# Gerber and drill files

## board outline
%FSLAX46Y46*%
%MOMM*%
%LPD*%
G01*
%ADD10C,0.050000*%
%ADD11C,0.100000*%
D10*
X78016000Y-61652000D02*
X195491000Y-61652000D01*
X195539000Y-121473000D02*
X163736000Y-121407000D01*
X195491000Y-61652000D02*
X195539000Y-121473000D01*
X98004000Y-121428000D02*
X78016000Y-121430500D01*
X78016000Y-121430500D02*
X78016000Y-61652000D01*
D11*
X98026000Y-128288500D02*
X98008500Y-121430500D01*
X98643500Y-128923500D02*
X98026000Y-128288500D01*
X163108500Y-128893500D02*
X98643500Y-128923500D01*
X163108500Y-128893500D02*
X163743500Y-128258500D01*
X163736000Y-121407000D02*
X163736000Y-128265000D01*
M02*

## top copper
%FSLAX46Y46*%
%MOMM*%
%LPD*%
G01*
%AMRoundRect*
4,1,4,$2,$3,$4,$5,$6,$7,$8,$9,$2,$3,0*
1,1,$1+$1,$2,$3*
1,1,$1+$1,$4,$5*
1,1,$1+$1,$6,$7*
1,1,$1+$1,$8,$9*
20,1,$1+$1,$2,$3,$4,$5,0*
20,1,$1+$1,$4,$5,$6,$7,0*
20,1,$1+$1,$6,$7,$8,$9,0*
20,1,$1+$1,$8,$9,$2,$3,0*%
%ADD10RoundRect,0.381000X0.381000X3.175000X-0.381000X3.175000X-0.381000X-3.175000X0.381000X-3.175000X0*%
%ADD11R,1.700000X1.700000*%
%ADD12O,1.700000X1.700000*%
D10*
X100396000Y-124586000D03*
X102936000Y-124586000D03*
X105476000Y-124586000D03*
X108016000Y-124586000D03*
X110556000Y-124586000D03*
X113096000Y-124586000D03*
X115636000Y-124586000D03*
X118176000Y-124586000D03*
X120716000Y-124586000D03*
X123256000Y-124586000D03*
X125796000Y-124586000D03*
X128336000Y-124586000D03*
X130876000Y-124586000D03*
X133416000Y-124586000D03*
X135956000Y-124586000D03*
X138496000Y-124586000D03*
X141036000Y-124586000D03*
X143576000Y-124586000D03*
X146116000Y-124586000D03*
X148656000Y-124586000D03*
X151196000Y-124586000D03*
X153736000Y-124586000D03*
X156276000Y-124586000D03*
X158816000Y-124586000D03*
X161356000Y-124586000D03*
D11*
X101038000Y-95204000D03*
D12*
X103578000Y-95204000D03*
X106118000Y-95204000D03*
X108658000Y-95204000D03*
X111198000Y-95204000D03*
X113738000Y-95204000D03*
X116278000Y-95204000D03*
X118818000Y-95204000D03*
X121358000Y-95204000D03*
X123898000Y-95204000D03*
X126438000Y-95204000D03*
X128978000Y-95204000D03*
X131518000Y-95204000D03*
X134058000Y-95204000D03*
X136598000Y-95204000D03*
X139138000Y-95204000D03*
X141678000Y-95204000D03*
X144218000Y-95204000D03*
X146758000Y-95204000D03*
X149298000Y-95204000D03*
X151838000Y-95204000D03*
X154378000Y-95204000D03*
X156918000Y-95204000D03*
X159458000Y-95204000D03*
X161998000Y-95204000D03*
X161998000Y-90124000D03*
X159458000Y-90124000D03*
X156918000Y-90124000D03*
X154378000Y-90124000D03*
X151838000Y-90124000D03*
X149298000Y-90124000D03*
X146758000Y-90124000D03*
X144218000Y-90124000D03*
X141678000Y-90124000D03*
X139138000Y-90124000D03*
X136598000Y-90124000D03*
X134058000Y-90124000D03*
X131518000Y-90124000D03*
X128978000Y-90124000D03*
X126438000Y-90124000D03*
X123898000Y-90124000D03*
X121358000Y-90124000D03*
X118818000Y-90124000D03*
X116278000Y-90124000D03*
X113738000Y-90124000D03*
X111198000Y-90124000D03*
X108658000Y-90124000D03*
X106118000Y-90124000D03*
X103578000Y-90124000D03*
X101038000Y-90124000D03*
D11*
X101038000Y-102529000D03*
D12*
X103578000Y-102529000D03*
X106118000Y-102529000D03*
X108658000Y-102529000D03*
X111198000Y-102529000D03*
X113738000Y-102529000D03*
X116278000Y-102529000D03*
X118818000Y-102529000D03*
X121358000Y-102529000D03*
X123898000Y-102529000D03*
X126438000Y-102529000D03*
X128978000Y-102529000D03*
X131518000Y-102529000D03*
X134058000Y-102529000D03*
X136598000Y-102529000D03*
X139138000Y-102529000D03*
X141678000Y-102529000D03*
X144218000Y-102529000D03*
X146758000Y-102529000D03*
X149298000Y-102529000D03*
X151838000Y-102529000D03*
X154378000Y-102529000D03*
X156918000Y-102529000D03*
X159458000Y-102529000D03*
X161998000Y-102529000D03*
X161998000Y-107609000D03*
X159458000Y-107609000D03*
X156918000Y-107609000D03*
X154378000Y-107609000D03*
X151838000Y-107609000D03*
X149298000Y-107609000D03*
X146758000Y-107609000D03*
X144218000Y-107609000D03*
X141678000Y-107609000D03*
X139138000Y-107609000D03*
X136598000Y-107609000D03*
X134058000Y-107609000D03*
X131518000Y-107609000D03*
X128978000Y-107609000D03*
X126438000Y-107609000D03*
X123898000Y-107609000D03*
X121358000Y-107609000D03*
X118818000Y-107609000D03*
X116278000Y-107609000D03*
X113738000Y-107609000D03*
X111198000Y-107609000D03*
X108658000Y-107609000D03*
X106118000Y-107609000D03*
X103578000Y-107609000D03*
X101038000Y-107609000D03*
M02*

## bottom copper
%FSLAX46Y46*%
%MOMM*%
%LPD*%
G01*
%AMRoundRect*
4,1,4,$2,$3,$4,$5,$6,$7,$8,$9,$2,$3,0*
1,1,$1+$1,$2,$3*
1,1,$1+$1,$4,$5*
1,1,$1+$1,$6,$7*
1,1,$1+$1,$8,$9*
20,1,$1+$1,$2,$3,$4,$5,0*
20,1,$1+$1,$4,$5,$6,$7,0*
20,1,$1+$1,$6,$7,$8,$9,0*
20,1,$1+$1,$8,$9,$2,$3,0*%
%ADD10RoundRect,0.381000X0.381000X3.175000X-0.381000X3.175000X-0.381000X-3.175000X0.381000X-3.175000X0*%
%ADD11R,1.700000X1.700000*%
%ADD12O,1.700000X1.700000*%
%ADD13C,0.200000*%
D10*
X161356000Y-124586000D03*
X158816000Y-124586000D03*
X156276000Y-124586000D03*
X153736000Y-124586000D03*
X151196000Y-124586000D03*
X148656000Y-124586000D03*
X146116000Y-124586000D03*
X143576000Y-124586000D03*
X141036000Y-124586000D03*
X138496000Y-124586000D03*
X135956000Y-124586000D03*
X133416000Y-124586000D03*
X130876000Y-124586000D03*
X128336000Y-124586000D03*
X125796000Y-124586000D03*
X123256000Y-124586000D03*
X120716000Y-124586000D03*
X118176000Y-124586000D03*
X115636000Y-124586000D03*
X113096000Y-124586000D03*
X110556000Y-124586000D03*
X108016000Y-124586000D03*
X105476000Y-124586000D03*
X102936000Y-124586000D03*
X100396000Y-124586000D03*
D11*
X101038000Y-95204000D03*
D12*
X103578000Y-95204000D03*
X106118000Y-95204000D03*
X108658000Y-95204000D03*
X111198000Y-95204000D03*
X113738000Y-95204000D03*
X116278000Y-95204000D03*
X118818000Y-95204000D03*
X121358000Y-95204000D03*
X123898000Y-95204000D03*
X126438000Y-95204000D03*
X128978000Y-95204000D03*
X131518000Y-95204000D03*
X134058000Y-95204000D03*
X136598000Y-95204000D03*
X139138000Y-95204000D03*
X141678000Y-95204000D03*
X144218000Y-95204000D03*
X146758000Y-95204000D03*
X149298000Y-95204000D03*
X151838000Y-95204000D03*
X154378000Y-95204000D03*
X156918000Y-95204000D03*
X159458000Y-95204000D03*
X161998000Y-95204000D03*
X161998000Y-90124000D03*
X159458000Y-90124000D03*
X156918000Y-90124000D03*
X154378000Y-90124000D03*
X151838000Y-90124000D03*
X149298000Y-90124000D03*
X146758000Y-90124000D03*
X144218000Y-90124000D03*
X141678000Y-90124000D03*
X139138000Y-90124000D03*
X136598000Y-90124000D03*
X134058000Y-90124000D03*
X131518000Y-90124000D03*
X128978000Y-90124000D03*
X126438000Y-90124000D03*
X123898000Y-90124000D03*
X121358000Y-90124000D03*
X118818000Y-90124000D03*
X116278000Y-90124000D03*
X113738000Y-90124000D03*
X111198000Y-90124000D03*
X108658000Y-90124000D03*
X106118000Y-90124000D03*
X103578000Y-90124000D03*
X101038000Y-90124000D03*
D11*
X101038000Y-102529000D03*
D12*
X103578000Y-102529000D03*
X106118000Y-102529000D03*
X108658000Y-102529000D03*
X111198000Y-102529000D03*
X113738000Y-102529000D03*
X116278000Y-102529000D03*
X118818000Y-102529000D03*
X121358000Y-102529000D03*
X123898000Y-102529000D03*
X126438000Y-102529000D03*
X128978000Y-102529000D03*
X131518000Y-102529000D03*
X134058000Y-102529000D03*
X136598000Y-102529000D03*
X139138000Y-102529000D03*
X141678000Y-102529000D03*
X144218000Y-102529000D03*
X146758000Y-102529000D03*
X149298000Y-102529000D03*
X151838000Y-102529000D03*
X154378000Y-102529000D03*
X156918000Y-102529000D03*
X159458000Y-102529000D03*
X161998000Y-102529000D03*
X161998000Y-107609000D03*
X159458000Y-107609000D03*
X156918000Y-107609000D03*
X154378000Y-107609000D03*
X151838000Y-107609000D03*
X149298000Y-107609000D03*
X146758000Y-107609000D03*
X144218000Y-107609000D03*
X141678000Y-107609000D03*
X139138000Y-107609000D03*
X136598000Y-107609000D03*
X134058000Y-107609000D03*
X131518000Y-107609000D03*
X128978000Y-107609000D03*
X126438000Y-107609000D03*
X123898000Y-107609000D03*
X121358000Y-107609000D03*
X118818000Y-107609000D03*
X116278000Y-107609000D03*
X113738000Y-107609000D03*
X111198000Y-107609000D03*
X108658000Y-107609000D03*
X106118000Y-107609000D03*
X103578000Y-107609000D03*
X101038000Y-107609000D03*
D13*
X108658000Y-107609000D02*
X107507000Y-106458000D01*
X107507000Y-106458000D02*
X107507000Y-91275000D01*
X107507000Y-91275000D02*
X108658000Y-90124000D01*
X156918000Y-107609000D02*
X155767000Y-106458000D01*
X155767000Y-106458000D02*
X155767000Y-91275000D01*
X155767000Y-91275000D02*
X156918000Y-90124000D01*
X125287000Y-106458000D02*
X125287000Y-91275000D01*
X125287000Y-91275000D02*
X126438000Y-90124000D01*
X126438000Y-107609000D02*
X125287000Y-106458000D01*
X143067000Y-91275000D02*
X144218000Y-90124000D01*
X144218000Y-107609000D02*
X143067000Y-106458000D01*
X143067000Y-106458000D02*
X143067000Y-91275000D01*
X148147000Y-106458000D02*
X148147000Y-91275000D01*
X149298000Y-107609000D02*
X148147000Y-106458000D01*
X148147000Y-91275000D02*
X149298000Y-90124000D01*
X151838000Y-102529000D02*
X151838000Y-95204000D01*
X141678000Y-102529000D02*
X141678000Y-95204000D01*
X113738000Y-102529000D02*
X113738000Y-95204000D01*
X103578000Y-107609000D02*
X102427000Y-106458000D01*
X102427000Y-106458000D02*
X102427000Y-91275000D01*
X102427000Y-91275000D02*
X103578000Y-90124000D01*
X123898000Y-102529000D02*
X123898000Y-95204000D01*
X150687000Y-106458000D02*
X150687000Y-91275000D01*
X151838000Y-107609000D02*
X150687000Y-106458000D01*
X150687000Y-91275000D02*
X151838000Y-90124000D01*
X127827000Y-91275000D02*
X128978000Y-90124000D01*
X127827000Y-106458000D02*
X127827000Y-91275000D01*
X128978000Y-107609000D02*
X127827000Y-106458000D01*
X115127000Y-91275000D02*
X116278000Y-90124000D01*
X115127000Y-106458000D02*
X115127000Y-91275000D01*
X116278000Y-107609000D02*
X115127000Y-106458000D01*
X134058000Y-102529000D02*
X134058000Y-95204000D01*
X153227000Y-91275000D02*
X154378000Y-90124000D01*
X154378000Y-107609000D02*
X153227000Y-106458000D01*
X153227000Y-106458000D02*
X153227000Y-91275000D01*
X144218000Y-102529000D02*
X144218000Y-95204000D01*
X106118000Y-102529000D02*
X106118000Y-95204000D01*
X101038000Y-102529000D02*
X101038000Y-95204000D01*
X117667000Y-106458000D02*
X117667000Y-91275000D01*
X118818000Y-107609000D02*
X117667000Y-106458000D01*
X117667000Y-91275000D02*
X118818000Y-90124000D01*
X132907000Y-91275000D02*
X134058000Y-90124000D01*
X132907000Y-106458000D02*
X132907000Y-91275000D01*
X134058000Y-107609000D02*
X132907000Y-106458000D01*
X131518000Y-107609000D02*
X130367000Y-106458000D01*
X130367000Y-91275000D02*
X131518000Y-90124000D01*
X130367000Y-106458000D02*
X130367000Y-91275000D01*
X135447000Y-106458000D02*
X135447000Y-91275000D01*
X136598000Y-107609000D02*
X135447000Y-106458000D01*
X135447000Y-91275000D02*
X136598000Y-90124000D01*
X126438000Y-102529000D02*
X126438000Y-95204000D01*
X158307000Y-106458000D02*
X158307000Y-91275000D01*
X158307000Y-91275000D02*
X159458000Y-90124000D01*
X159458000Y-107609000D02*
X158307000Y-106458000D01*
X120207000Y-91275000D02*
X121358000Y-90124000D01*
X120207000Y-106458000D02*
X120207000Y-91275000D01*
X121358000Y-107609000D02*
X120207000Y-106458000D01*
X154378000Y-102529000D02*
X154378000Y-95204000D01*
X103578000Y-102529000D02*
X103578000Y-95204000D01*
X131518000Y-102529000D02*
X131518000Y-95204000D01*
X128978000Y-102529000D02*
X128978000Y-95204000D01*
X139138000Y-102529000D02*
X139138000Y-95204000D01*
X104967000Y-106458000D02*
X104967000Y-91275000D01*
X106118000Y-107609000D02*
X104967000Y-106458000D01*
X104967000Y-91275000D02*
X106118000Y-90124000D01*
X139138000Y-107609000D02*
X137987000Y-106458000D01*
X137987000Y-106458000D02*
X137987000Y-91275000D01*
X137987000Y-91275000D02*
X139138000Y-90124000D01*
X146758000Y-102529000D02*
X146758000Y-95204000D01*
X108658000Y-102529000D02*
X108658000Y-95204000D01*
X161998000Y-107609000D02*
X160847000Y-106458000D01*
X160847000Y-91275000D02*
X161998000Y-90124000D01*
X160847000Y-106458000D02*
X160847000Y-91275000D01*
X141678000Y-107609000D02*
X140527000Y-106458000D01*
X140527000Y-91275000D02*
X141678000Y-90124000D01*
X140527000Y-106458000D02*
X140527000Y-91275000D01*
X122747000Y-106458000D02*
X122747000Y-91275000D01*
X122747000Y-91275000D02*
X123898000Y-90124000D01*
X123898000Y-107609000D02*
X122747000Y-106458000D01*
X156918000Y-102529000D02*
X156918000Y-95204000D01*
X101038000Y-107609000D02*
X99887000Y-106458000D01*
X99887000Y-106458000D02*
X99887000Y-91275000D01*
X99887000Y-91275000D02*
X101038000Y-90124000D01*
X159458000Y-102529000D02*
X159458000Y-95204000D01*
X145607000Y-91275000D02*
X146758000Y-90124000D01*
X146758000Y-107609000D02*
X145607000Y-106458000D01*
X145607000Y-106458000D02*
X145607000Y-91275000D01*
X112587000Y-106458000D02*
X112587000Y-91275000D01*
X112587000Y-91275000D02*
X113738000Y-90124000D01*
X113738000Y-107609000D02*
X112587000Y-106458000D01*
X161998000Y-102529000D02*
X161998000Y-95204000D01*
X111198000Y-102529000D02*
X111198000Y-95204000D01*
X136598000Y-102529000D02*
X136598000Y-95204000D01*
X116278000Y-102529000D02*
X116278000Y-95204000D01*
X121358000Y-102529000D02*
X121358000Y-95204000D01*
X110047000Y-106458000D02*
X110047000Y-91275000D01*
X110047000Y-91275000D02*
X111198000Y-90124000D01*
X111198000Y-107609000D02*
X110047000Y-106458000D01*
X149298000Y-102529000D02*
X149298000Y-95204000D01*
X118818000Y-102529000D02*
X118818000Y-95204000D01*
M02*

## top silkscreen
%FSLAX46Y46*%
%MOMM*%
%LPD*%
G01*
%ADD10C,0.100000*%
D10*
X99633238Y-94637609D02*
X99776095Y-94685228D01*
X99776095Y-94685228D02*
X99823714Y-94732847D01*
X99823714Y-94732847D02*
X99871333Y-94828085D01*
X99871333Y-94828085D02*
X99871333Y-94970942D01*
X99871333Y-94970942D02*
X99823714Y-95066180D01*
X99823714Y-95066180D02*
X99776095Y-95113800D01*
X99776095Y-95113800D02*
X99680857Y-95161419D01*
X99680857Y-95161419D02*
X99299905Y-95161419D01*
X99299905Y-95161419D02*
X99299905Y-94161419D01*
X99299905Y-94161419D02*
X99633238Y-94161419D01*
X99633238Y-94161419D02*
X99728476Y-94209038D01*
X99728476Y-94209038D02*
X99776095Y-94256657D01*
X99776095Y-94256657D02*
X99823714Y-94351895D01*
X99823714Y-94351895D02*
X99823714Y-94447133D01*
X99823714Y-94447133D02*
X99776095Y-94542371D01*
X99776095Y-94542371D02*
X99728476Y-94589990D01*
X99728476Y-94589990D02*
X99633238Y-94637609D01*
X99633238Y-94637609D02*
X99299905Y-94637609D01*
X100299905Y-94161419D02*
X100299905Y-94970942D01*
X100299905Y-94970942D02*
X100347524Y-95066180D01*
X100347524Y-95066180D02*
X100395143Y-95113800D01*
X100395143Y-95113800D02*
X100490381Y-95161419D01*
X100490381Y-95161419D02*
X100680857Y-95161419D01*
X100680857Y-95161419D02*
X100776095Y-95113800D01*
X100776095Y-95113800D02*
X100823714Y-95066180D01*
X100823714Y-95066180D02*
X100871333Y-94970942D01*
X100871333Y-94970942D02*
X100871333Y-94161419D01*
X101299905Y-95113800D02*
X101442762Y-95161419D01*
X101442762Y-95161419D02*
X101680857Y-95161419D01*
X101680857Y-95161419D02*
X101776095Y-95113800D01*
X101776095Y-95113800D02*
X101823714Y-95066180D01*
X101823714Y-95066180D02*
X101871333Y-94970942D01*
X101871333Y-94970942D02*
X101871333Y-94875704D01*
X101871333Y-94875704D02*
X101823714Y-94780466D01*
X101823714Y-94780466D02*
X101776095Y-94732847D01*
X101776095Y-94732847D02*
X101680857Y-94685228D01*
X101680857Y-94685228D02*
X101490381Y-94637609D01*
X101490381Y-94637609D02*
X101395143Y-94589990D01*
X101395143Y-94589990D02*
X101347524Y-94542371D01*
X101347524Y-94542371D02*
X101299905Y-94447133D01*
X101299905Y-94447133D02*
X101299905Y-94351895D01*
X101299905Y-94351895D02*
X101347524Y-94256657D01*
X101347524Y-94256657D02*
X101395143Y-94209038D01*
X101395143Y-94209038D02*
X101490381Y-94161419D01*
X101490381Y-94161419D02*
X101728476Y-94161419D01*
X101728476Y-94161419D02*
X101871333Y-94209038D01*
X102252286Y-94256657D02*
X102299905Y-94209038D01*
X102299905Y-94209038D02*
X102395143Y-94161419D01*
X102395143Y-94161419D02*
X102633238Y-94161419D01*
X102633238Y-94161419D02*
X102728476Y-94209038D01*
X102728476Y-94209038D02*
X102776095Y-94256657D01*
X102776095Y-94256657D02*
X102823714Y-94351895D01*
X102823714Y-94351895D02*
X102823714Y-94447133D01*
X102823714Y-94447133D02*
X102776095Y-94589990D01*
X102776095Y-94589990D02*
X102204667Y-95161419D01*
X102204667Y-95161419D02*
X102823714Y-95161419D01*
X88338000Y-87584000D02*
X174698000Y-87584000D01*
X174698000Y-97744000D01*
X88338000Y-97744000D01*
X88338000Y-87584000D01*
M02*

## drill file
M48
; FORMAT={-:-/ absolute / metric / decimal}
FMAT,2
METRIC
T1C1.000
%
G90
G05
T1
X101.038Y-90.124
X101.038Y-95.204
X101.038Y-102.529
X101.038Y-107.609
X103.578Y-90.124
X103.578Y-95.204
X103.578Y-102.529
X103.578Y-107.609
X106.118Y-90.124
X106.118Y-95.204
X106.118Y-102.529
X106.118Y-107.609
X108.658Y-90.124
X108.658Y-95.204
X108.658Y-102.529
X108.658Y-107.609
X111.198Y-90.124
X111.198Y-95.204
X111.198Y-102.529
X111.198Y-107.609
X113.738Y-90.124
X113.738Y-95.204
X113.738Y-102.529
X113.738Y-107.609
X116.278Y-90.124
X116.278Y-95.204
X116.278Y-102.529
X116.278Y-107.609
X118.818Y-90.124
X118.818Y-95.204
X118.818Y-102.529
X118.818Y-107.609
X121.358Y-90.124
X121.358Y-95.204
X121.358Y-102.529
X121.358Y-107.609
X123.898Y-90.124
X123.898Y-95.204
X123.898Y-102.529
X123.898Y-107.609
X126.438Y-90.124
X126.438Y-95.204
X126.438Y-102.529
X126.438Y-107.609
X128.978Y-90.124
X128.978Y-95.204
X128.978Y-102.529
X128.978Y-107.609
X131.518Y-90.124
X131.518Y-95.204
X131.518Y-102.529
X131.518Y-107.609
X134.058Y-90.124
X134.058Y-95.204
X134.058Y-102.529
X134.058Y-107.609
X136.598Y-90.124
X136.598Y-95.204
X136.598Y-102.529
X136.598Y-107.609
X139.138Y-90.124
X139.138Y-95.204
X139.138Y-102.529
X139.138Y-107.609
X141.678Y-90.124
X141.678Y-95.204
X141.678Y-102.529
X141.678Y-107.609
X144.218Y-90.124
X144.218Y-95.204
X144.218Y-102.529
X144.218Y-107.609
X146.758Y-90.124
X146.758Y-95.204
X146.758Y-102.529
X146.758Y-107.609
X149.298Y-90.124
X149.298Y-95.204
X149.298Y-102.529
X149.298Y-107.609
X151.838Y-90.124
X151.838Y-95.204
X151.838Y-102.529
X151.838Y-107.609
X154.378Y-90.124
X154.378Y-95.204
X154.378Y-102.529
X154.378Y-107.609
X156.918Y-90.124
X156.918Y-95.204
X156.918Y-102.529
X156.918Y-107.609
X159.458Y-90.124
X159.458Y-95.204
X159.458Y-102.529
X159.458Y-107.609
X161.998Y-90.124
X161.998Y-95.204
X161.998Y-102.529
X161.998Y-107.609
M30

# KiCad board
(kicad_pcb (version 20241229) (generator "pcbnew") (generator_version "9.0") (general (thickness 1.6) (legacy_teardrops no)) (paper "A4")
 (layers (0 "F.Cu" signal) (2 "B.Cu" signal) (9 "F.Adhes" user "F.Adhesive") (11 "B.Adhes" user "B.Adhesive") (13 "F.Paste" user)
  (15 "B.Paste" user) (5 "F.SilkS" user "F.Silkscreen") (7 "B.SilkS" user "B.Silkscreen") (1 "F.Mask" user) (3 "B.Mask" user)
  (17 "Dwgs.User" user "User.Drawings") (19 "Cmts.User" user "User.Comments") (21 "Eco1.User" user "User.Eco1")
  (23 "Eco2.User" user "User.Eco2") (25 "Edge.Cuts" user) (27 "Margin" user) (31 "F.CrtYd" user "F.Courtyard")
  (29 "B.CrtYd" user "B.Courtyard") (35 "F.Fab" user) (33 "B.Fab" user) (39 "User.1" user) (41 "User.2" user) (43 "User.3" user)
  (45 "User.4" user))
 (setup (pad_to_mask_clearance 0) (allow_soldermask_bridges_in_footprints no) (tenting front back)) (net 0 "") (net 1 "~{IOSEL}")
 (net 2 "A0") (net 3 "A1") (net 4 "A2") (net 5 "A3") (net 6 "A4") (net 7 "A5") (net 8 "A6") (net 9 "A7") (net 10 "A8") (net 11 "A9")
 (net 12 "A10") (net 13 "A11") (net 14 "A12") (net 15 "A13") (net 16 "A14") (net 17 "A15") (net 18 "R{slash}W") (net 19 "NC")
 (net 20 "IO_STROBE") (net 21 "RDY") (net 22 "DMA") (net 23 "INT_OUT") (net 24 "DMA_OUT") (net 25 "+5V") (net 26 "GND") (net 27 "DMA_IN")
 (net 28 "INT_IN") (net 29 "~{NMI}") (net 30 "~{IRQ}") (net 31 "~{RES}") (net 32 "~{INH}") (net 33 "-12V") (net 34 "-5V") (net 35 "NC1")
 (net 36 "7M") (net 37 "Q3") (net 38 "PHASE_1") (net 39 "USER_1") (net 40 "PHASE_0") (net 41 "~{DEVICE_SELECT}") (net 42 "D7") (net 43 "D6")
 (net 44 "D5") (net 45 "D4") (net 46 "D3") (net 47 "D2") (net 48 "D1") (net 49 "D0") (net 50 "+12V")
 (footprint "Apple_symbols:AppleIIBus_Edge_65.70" (layer "F.Cu") (at 130.876 124.586)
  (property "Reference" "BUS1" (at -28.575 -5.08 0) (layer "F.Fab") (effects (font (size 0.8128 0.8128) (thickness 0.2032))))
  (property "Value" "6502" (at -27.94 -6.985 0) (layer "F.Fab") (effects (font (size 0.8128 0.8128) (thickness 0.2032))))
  (fp_line (start -32.85 3.7025) (end -32.8675 -3.1555) (stroke (width 0.1) (type solid)) (layer "Edge.Cuts"))
  (fp_line (start -32.2325 4.3375) (end -32.85 3.7025) (stroke (width 0.1) (type default)) (layer "Edge.Cuts"))
  (fp_line (start 32.2325 4.3075) (end -32.2325 4.3375) (stroke (width 0.1) (type solid)) (layer "Edge.Cuts"))
  (fp_line (start 32.2325 4.3075) (end 32.8675 3.6725) (stroke (width 0.1) (type default)) (layer "Edge.Cuts"))
  (fp_line (start 32.86 -3.179) (end 32.86 3.679) (stroke (width 0.1) (type solid)) (layer "Edge.Cuts"))
  (pad "1" connect roundrect (at -30.48 0 180) (size 1.524 7.112) (layers "F.Cu" "F.Mask") (roundrect_rratio 0.25) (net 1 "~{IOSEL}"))
  (pad "2" connect roundrect (at -27.94 0 180) (size 1.524 7.112) (layers "F.Cu" "F.Mask") (roundrect_rratio 0.25) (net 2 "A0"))
  (pad "3" connect roundrect (at -25.4 0 180) (size 1.524 7.112) (layers "F.Cu" "F.Mask") (roundrect_rratio 0.25) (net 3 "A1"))
  (pad "4" connect roundrect (at -22.86 0 180) (size 1.524 7.112) (layers "F.Cu" "F.Mask") (roundrect_rratio 0.25) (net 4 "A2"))
  (pad "5" connect roundrect (at -20.32 0 180) (size 1.524 7.112) (layers "F.Cu" "F.Mask") (roundrect_rratio 0.25) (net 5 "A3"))
  (pad "6" connect roundrect (at -17.78 0 180) (size 1.524 7.112) (layers "F.Cu" "F.Mask") (roundrect_rratio 0.25) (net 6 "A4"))
  (pad "7" connect roundrect (at -15.24 0 180) (size 1.524 7.112) (layers "F.Cu" "F.Mask") (roundrect_rratio 0.25) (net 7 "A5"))
  (pad "8" connect roundrect (at -12.7 0 180) (size 1.524 7.112) (layers "F.Cu" "F.Mask") (roundrect_rratio 0.25) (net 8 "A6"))
  (pad "9" connect roundrect (at -10.16 0 180) (size 1.524 7.112) (layers "F.Cu" "F.Mask") (roundrect_rratio 0.25) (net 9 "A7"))
  (pad "10" connect roundrect (at -7.62 0 180) (size 1.524 7.112) (layers "F.Cu" "F.Mask") (roundrect_rratio 0.25) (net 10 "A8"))
  (pad "11" connect roundrect (at -5.08 0 180) (size 1.524 7.112) (layers "F.Cu" "F.Mask") (roundrect_rratio 0.25) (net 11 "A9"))
  (pad "12" connect roundrect (at -2.54 0 180) (size 1.524 7.112) (layers "F.Cu" "F.Mask") (roundrect_rratio 0.25) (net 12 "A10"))
  (pad "13" connect roundrect (at 0 0 180) (size 1.524 7.112) (layers "F.Cu" "F.Mask") (roundrect_rratio 0.25) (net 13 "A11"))
  (pad "14" connect roundrect (at 2.54 0 180) (size 1.524 7.112) (layers "F.Cu" "F.Mask") (roundrect_rratio 0.25) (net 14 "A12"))
  (pad "15" connect roundrect (at 5.08 0 180) (size 1.524 7.112) (layers "F.Cu" "F.Mask") (roundrect_rratio 0.25) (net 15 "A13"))
  (pad "16" connect roundrect (at 7.62 0 180) (size 1.524 7.112) (layers "F.Cu" "F.Mask") (roundrect_rratio 0.25) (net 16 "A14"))
  (pad "17" connect roundrect (at 10.16 0 180) (size 1.524 7.112) (layers "F.Cu" "F.Mask") (roundrect_rratio 0.25) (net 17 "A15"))
  (pad "18" connect roundrect (at 12.7 0 180) (size 1.524 7.112) (layers "F.Cu" "F.Mask") (roundrect_rratio 0.25) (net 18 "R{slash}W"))
  (pad "19" connect roundrect (at 15.24 0 180) (size 1.524 7.112) (layers "F.Cu" "F.Mask") (roundrect_rratio 0.25) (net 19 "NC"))
  (pad "20" connect roundrect (at 17.78 0 180) (size 1.524 7.112) (layers "F.Cu" "F.Mask") (roundrect_rratio 0.25) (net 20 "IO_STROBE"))
  (pad "21" connect roundrect (at 20.32 0 180) (size 1.524 7.112) (layers "F.Cu" "F.Mask") (roundrect_rratio 0.25) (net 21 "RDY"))
  (pad "22" connect roundrect (at 22.86 0 180) (size 1.524 7.112) (layers "F.Cu" "F.Mask") (roundrect_rratio 0.25) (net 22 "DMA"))
  (pad "23" connect roundrect (at 25.4 0 180) (size 1.524 7.112) (layers "F.Cu" "F.Mask") (roundrect_rratio 0.25) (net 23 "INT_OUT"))
  (pad "24" connect roundrect (at 27.94 0 180) (size 1.524 7.112) (layers "F.Cu" "F.Mask") (roundrect_rratio 0.25) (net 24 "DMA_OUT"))
  (pad "25" connect roundrect (at 30.48 0 180) (size 1.524 7.112) (layers "F.Cu" "F.Mask") (roundrect_rratio 0.25) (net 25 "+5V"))
  (pad "26" connect roundrect (at 30.48 0 180) (size 1.524 7.112) (layers "B.Cu" "B.Mask") (roundrect_rratio 0.25) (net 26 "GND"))
  (pad "27" connect roundrect (at 27.94 0 180) (size 1.524 7.112) (layers "B.Cu" "B.Mask") (roundrect_rratio 0.25) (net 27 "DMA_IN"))
  (pad "28" connect roundrect (at 25.4 0 180) (size 1.524 7.112) (layers "B.Cu" "B.Mask") (roundrect_rratio 0.25) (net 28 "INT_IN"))
  (pad "29" connect roundrect (at 22.86 0 180) (size 1.524 7.112) (layers "B.Cu" "B.Mask") (roundrect_rratio 0.25) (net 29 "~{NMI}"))
  (pad "30" connect roundrect (at 20.32 0 180) (size 1.524 7.112) (layers "B.Cu" "B.Mask") (roundrect_rratio 0.25) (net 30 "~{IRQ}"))
  (pad "31" connect roundrect (at 17.78 0 180) (size 1.524 7.112) (layers "B.Cu" "B.Mask") (roundrect_rratio 0.25) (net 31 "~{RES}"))
  (pad "32" connect roundrect (at 15.24 0 180) (size 1.524 7.112) (layers "B.Cu" "B.Mask") (roundrect_rratio 0.25) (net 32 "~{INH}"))
  (pad "33" connect roundrect (at 12.7 0 180) (size 1.524 7.112) (layers "B.Cu" "B.Mask") (roundrect_rratio 0.25) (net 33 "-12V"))
  (pad "34" connect roundrect (at 10.16 0 180) (size 1.524 7.112) (layers "B.Cu" "B.Mask") (roundrect_rratio 0.25) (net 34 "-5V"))
  (pad "35" connect roundrect (at 7.62 0 180) (size 1.524 7.112) (layers "B.Cu" "B.Mask") (roundrect_rratio 0.25) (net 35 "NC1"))
  (pad "36" connect roundrect (at 5.08 0 180) (size 1.524 7.112) (layers "B.Cu" "B.Mask") (roundrect_rratio 0.25) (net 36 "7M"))
  (pad "37" connect roundrect (at 2.54 0 180) (size 1.524 7.112) (layers "B.Cu" "B.Mask") (roundrect_rratio 0.25) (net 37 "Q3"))
  (pad "38" connect roundrect (at 0 0 180) (size 1.524 7.112) (layers "B.Cu" "B.Mask") (roundrect_rratio 0.25) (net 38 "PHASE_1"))
  (pad "39" connect roundrect (at -2.54 0 180) (size 1.524 7.112) (layers "B.Cu" "B.Mask") (roundrect_rratio 0.25) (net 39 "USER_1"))
  (pad "40" connect roundrect (at -5.08 0 180) (size 1.524 7.112) (layers "B.Cu" "B.Mask") (roundrect_rratio 0.25) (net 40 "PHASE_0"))
  (pad "41" connect roundrect (at -7.62 0 180) (size 1.524 7.112) (layers "B.Cu" "B.Mask") (roundrect_rratio 0.25)
   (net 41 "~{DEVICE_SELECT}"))
  (pad "42" connect roundrect (at -10.16 0 180) (size 1.524 7.112) (layers "B.Cu" "B.Mask") (roundrect_rratio 0.25) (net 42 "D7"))
  (pad "43" connect roundrect (at -12.7 0 180) (size 1.524 7.112) (layers "B.Cu" "B.Mask") (roundrect_rratio 0.25) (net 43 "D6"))
  (pad "44" connect roundrect (at -15.24 0 180) (size 1.524 7.112) (layers "B.Cu" "B.Mask") (roundrect_rratio 0.25) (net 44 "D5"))
  (pad "45" connect roundrect (at -17.78 0 180) (size 1.524 7.112) (layers "B.Cu" "B.Mask") (roundrect_rratio 0.25) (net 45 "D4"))
  (pad "46" connect roundrect (at -20.32 0 180) (size 1.524 7.112) (layers "B.Cu" "B.Mask") (roundrect_rratio 0.25) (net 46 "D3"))
  (pad "47" connect roundrect (at -22.86 0 180) (size 1.524 7.112) (layers "B.Cu" "B.Mask") (roundrect_rratio 0.25) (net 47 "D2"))
  (pad "48" connect roundrect (at -25.4 0 180) (size 1.524 7.112) (layers "B.Cu" "B.Mask") (roundrect_rratio 0.25) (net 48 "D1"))
  (pad "49" connect roundrect (at -27.94 0 180) (size 1.524 7.112) (layers "B.Cu" "B.Mask") (roundrect_rratio 0.25) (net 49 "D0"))
  (pad "50" connect roundrect (at -30.48 0 180) (size 1.524 7.112) (layers "B.Cu" "B.Mask") (roundrect_rratio 0.25) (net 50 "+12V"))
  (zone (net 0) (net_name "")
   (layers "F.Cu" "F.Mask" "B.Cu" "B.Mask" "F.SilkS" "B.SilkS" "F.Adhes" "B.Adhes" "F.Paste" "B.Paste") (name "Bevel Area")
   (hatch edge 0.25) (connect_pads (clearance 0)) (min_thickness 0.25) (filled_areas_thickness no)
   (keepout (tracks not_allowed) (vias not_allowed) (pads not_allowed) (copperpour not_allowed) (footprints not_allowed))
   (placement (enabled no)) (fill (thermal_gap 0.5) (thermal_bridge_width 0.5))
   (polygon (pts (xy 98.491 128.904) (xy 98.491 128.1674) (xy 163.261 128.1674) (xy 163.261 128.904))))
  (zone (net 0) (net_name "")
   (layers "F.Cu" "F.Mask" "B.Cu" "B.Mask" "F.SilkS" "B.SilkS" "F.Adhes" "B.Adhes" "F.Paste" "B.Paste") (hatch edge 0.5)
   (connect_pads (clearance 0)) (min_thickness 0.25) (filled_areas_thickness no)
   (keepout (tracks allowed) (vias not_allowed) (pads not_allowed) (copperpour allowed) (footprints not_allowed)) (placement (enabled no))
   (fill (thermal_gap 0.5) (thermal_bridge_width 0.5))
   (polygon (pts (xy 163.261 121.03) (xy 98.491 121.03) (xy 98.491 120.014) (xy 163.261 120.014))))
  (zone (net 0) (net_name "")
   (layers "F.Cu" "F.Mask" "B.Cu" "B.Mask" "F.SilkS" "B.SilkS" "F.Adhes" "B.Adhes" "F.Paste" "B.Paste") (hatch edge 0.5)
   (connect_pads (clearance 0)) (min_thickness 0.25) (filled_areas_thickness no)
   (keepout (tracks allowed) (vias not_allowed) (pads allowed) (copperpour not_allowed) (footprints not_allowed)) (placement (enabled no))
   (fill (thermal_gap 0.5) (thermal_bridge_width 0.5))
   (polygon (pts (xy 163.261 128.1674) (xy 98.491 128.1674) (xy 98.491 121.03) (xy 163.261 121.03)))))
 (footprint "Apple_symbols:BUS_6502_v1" (layer "F.Cu") (at 101.038 95.204)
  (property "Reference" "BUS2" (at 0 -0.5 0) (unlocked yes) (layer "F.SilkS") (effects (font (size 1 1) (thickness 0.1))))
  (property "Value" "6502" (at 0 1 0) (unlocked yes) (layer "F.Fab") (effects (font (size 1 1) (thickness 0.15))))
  (fp_rect (start -12.7 -7.62) (end 73.66 2.54) (stroke (width 0.1) (type default)) (fill no) (layer "F.SilkS"))
  (pad "1" thru_hole rect (at 0 0 90) (size 1.7 1.7) (drill 1) (layers "*.Cu" "*.Mask") (remove_unused_layers no) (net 1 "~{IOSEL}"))
  (pad "2" thru_hole oval (at 2.54 0 90) (size 1.7 1.7) (drill 1) (layers "*.Cu" "*.Mask") (remove_unused_layers no) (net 2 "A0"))
  (pad "3" thru_hole oval (at 5.08 0 90) (size 1.7 1.7) (drill 1) (layers "*.Cu" "*.Mask") (remove_unused_layers no) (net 3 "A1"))
  (pad "4" thru_hole oval (at 7.62 0 90) (size 1.7 1.7) (drill 1) (layers "*.Cu" "*.Mask") (remove_unused_layers no) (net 4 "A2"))
  (pad "5" thru_hole oval (at 10.16 0 90) (size 1.7 1.7) (drill 1) (layers "*.Cu" "*.Mask") (remove_unused_layers no) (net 5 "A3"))
  (pad "6" thru_hole oval (at 12.7 0 90) (size 1.7 1.7) (drill 1) (layers "*.Cu" "*.Mask") (remove_unused_layers no) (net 6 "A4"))
  (pad "7" thru_hole oval (at 15.24 0 90) (size 1.7 1.7) (drill 1) (layers "*.Cu" "*.Mask") (remove_unused_layers no) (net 7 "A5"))
  (pad "8" thru_hole oval (at 17.78 0 90) (size 1.7 1.7) (drill 1) (layers "*.Cu" "*.Mask") (remove_unused_layers no) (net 8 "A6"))
  (pad "9" thru_hole oval (at 20.32 0 90) (size 1.7 1.7) (drill 1) (layers "*.Cu" "*.Mask") (remove_unused_layers no) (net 9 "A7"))
  (pad "10" thru_hole oval (at 22.86 0 90) (size 1.7 1.7) (drill 1) (layers "*.Cu" "*.Mask") (remove_unused_layers no) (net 10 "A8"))
  (pad "11" thru_hole oval (at 25.4 0 90) (size 1.7 1.7) (drill 1) (layers "*.Cu" "*.Mask") (remove_unused_layers no) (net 11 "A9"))
  (pad "12" thru_hole oval (at 27.94 0 90) (size 1.7 1.7) (drill 1) (layers "*.Cu" "*.Mask") (remove_unused_layers no) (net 12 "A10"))
  (pad "13" thru_hole oval (at 30.48 0 90) (size 1.7 1.7) (drill 1) (layers "*.Cu" "*.Mask") (remove_unused_layers no) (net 13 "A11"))
  (pad "14" thru_hole oval (at 33.02 0 90) (size 1.7 1.7) (drill 1) (layers "*.Cu" "*.Mask") (remove_unused_layers no) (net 14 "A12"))
  (pad "15" thru_hole oval (at 35.56 0 90) (size 1.7 1.7) (drill 1) (layers "*.Cu" "*.Mask") (remove_unused_layers no) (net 15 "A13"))
  (pad "16" thru_hole oval (at 38.1 0 90) (size 1.7 1.7) (drill 1) (layers "*.Cu" "*.Mask") (remove_unused_layers no) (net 16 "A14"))
  (pad "17" thru_hole oval (at 40.64 0 90) (size 1.7 1.7) (drill 1) (layers "*.Cu" "*.Mask") (remove_unused_layers no) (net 17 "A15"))
  (pad "18" thru_hole oval (at 43.18 0 90) (size 1.7 1.7) (drill 1) (layers "*.Cu" "*.Mask") (remove_unused_layers no) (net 18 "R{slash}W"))
  (pad "19" thru_hole oval (at 45.72 0 90) (size 1.7 1.7) (drill 1) (layers "*.Cu" "*.Mask") (remove_unused_layers no) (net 19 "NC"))
  (pad "20" thru_hole oval (at 48.26 0 90) (size 1.7 1.7) (drill 1) (layers "*.Cu" "*.Mask") (remove_unused_layers no) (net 20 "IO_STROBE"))
  (pad "21" thru_hole oval (at 50.8 0 90) (size 1.7 1.7) (drill 1) (layers "*.Cu" "*.Mask") (remove_unused_layers no) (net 21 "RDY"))
  (pad "22" thru_hole oval (at 53.34 0 90) (size 1.7 1.7) (drill 1) (layers "*.Cu" "*.Mask") (remove_unused_layers no) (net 22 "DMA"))
  (pad "23" thru_hole oval (at 55.88 0 90) (size 1.7 1.7) (drill 1) (layers "*.Cu" "*.Mask") (remove_unused_layers no) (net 23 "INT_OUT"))
  (pad "24" thru_hole oval (at 58.42 0 90) (size 1.7 1.7) (drill 1) (layers "*.Cu" "*.Mask") (remove_unused_layers no) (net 24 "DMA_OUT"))
  (pad "25" thru_hole oval (at 60.96 0 90) (size 1.7 1.7) (drill 1) (layers "*.Cu" "*.Mask") (remove_unused_layers no) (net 25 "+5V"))
  (pad "26" thru_hole oval (at 60.96 -5.08 90) (size 1.7 1.7) (drill 1) (layers "*.Cu" "*.Mask") (remove_unused_layers no) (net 26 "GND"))
  (pad "27" thru_hole oval (at 58.42 -5.08 90) (size 1.7 1.7) (drill 1) (layers "*.Cu" "*.Mask") (remove_unused_layers no) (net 27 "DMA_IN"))
  (pad "28" thru_hole oval (at 55.88 -5.08 90) (size 1.7 1.7) (drill 1) (layers "*.Cu" "*.Mask") (remove_unused_layers no) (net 28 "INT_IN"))
  (pad "29" thru_hole oval (at 53.34 -5.08 90) (size 1.7 1.7) (drill 1) (layers "*.Cu" "*.Mask") (remove_unused_layers no) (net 29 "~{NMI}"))
  (pad "30" thru_hole oval (at 50.8 -5.08 90) (size 1.7 1.7) (drill 1) (layers "*.Cu" "*.Mask") (remove_unused_layers no) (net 30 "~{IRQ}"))
  (pad "31" thru_hole oval (at 48.26 -5.08 90) (size 1.7 1.7) (drill 1) (layers "*.Cu" "*.Mask") (remove_unused_layers no) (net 31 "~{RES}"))
  (pad "32" thru_hole oval (at 45.72 -5.08 90) (size 1.7 1.7) (drill 1) (layers "*.Cu" "*.Mask") (remove_unused_layers no) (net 32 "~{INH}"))
  (pad "33" thru_hole oval (at 43.18 -5.08 90) (size 1.7 1.7) (drill 1) (layers "*.Cu" "*.Mask") (remove_unused_layers no) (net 33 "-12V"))
  (pad "34" thru_hole oval (at 40.64 -5.08 90) (size 1.7 1.7) (drill 1) (layers "*.Cu" "*.Mask") (remove_unused_layers no) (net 34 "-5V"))
  (pad "35" thru_hole oval (at 38.1 -5.08 90) (size 1.7 1.7) (drill 1) (layers "*.Cu" "*.Mask") (remove_unused_layers no) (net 35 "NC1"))
  (pad "36" thru_hole oval (at 35.56 -5.08 90) (size 1.7 1.7) (drill 1) (layers "*.Cu" "*.Mask") (remove_unused_layers no) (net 36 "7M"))
  (pad "37" thru_hole oval (at 33.02 -5.08 90) (size 1.7 1.7) (drill 1) (layers "*.Cu" "*.Mask") (remove_unused_layers no) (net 37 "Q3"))
  (pad "38" thru_hole oval (at 30.48 -5.08 90) (size 1.7 1.7) (drill 1) (layers "*.Cu" "*.Mask") (remove_unused_layers no)
   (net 38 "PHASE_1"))
  (pad "39" thru_hole oval (at 27.94 -5.08 90) (size 1.7 1.7) (drill 1) (layers "*.Cu" "*.Mask") (remove_unused_layers no) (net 39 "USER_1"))
  (pad "40" thru_hole oval (at 25.4 -5.08 90) (size 1.7 1.7) (drill 1) (layers "*.Cu" "*.Mask") (remove_unused_layers no) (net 40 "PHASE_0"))
  (pad "41" thru_hole oval (at 22.86 -5.08 90) (size 1.7 1.7) (drill 1) (layers "*.Cu" "*.Mask") (remove_unused_layers no)
   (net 41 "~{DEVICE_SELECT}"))
  (pad "42" thru_hole oval (at 20.32 -5.08 90) (size 1.7 1.7) (drill 1) (layers "*.Cu" "*.Mask") (remove_unused_layers no) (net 42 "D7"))
  (pad "43" thru_hole oval (at 17.78 -5.08 90) (size 1.7 1.7) (drill 1) (layers "*.Cu" "*.Mask") (remove_unused_layers no) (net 43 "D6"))
  (pad "44" thru_hole oval (at 15.24 -5.08 90) (size 1.7 1.7) (drill 1) (layers "*.Cu" "*.Mask") (remove_unused_layers no) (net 44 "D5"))
  (pad "45" thru_hole oval (at 12.7 -5.08 90) (size 1.7 1.7) (drill 1) (layers "*.Cu" "*.Mask") (remove_unused_layers no) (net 45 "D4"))
  (pad "46" thru_hole oval (at 10.16 -5.08 90) (size 1.7 1.7) (drill 1) (layers "*.Cu" "*.Mask") (remove_unused_layers no) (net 46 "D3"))
  (pad "47" thru_hole oval (at 7.62 -5.08 90) (size 1.7 1.7) (drill 1) (layers "*.Cu" "*.Mask") (remove_unused_layers no) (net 47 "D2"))
  (pad "48" thru_hole oval (at 5.08 -5.08 90) (size 1.7 1.7) (drill 1) (layers "*.Cu" "*.Mask") (remove_unused_layers no) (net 48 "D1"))
  (pad "49" thru_hole oval (at 2.54 -5.08 90) (size 1.7 1.7) (drill 1) (layers "*.Cu" "*.Mask") (remove_unused_layers no) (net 49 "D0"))
  (pad "50" thru_hole oval (at 0 -5.08 90) (size 1.7 1.7) (drill 1) (layers "*.Cu" "*.Mask") (remove_unused_layers no) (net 50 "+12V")))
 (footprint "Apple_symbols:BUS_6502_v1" (layer "B.Cu") (at 101.038 102.529)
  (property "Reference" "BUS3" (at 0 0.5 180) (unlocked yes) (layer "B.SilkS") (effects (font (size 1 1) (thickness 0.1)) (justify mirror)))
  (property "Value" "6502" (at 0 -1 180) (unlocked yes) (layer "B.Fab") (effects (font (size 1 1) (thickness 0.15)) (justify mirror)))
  (pad "1" thru_hole rect (at 0 0 270) (size 1.7 1.7) (drill 1) (layers "*.Cu" "*.Mask") (remove_unused_layers no) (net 1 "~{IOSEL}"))
  (pad "2" thru_hole oval (at 2.54 0 270) (size 1.7 1.7) (drill 1) (layers "*.Cu" "*.Mask") (remove_unused_layers no) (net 2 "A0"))
  (pad "3" thru_hole oval (at 5.08 0 270) (size 1.7 1.7) (drill 1) (layers "*.Cu" "*.Mask") (remove_unused_layers no) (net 3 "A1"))
  (pad "4" thru_hole oval (at 7.62 0 270) (size 1.7 1.7) (drill 1) (layers "*.Cu" "*.Mask") (remove_unused_layers no) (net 4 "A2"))
  (pad "5" thru_hole oval (at 10.16 0 270) (size 1.7 1.7) (drill 1) (layers "*.Cu" "*.Mask") (remove_unused_layers no) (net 5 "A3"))
  (pad "6" thru_hole oval (at 12.7 0 270) (size 1.7 1.7) (drill 1) (layers "*.Cu" "*.Mask") (remove_unused_layers no) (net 6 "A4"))
  (pad "7" thru_hole oval (at 15.24 0 270) (size 1.7 1.7) (drill 1) (layers "*.Cu" "*.Mask") (remove_unused_layers no) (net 7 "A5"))
  (pad "8" thru_hole oval (at 17.78 0 270) (size 1.7 1.7) (drill 1) (layers "*.Cu" "*.Mask") (remove_unused_layers no) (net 8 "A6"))
  (pad "9" thru_hole oval (at 20.32 0 270) (size 1.7 1.7) (drill 1) (layers "*.Cu" "*.Mask") (remove_unused_layers no) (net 9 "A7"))
  (pad "10" thru_hole oval (at 22.86 0 270) (size 1.7 1.7) (drill 1) (layers "*.Cu" "*.Mask") (remove_unused_layers no) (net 10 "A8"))
  (pad "11" thru_hole oval (at 25.4 0 270) (size 1.7 1.7) (drill 1) (layers "*.Cu" "*.Mask") (remove_unused_layers no) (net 11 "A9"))
  (pad "12" thru_hole oval (at 27.94 0 270) (size 1.7 1.7) (drill 1) (layers "*.Cu" "*.Mask") (remove_unused_layers no) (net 12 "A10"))
  (pad "13" thru_hole oval (at 30.48 0 270) (size 1.7 1.7) (drill 1) (layers "*.Cu" "*.Mask") (remove_unused_layers no) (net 13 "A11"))
  (pad "14" thru_hole oval (at 33.02 0 270) (size 1.7 1.7) (drill 1) (layers "*.Cu" "*.Mask") (remove_unused_layers no) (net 14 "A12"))
  (pad "15" thru_hole oval (at 35.56 0 270) (size 1.7 1.7) (drill 1) (layers "*.Cu" "*.Mask") (remove_unused_layers no) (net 15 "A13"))
  (pad "16" thru_hole oval (at 38.1 0 270) (size 1.7 1.7) (drill 1) (layers "*.Cu" "*.Mask") (remove_unused_layers no) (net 16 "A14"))
  (pad "17" thru_hole oval (at 40.64 0 270) (size 1.7 1.7) (drill 1) (layers "*.Cu" "*.Mask") (remove_unused_layers no) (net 17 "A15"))
  (pad "18" thru_hole oval (at 43.18 0 270) (size 1.7 1.7) (drill 1) (layers "*.Cu" "*.Mask") (remove_unused_layers no) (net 18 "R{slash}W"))
  (pad "19" thru_hole oval (at 45.72 0 270) (size 1.7 1.7) (drill 1) (layers "*.Cu" "*.Mask") (remove_unused_layers no) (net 19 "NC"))
  (pad "20" thru_hole oval (at 48.26 0 270) (size 1.7 1.7) (drill 1) (layers "*.Cu" "*.Mask") (remove_unused_layers no) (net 20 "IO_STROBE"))
  (pad "21" thru_hole oval (at 50.8 0 270) (size 1.7 1.7) (drill 1) (layers "*.Cu" "*.Mask") (remove_unused_layers no) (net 21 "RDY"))
  (pad "22" thru_hole oval (at 53.34 0 270) (size 1.7 1.7) (drill 1) (layers "*.Cu" "*.Mask") (remove_unused_layers no) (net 22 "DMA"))
  (pad "23" thru_hole oval (at 55.88 0 270) (size 1.7 1.7) (drill 1) (layers "*.Cu" "*.Mask") (remove_unused_layers no) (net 23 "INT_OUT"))
  (pad "24" thru_hole oval (at 58.42 0 270) (size 1.7 1.7) (drill 1) (layers "*.Cu" "*.Mask") (remove_unused_layers no) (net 24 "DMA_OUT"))
  (pad "25" thru_hole oval (at 60.96 0 270) (size 1.7 1.7) (drill 1) (layers "*.Cu" "*.Mask") (remove_unused_layers no) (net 25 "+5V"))
  (pad "26" thru_hole oval (at 60.96 5.08 270) (size 1.7 1.7) (drill 1) (layers "*.Cu" "*.Mask") (remove_unused_layers no) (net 26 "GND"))
  (pad "27" thru_hole oval (at 58.42 5.08 270) (size 1.7 1.7) (drill 1) (layers "*.Cu" "*.Mask") (remove_unused_layers no) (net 27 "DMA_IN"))
  (pad "28" thru_hole oval (at 55.88 5.08 270) (size 1.7 1.7) (drill 1) (layers "*.Cu" "*.Mask") (remove_unused_layers no) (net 28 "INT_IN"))
  (pad "29" thru_hole oval (at 53.34 5.08 270) (size 1.7 1.7) (drill 1) (layers "*.Cu" "*.Mask") (remove_unused_layers no) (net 29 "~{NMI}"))
  (pad "30" thru_hole oval (at 50.8 5.08 270) (size 1.7 1.7) (drill 1) (layers "*.Cu" "*.Mask") (remove_unused_layers no) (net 30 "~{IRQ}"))
  (pad "31" thru_hole oval (at 48.26 5.08 270) (size 1.7 1.7) (drill 1) (layers "*.Cu" "*.Mask") (remove_unused_layers no) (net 31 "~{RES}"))
  (pad "32" thru_hole oval (at 45.72 5.08 270) (size 1.7 1.7) (drill 1) (layers "*.Cu" "*.Mask") (remove_unused_layers no) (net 32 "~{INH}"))
  (pad "33" thru_hole oval (at 43.18 5.08 270) (size 1.7 1.7) (drill 1) (layers "*.Cu" "*.Mask") (remove_unused_layers no) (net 33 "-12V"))
  (pad "34" thru_hole oval (at 40.64 5.08 270) (size 1.7 1.7) (drill 1) (layers "*.Cu" "*.Mask") (remove_unused_layers no) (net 34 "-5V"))
  (pad "35" thru_hole oval (at 38.1 5.08 270) (size 1.7 1.7) (drill 1) (layers "*.Cu" "*.Mask") (remove_unused_layers no) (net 35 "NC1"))
  (pad "36" thru_hole oval (at 35.56 5.08 270) (size 1.7 1.7) (drill 1) (layers "*.Cu" "*.Mask") (remove_unused_layers no) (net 36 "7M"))
  (pad "37" thru_hole oval (at 33.02 5.08 270) (size 1.7 1.7) (drill 1) (layers "*.Cu" "*.Mask") (remove_unused_layers no) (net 37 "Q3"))
  (pad "38" thru_hole oval (at 30.48 5.08 270) (size 1.7 1.7) (drill 1) (layers "*.Cu" "*.Mask") (remove_unused_layers no)
   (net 38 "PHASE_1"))
  (pad "39" thru_hole oval (at 27.94 5.08 270) (size 1.7 1.7) (drill 1) (layers "*.Cu" "*.Mask") (remove_unused_layers no) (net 39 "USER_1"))
  (pad "40" thru_hole oval (at 25.4 5.08 270) (size 1.7 1.7) (drill 1) (layers "*.Cu" "*.Mask") (remove_unused_layers no) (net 40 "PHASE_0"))
  (pad "41" thru_hole oval (at 22.86 5.08 270) (size 1.7 1.7) (drill 1) (layers "*.Cu" "*.Mask") (remove_unused_layers no)
   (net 41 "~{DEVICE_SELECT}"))
  (pad "42" thru_hole oval (at 20.32 5.08 270) (size 1.7 1.7) (drill 1) (layers "*.Cu" "*.Mask") (remove_unused_layers no) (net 42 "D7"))
  (pad "43" thru_hole oval (at 17.78 5.08 270) (size 1.7 1.7) (drill 1) (layers "*.Cu" "*.Mask") (remove_unused_layers no) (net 43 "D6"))
  (pad "44" thru_hole oval (at 15.24 5.08 270) (size 1.7 1.7) (drill 1) (layers "*.Cu" "*.Mask") (remove_unused_layers no) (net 44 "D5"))
  (pad "45" thru_hole oval (at 12.7 5.08 270) (size 1.7 1.7) (drill 1) (layers "*.Cu" "*.Mask") (remove_unused_layers no) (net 45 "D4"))
  (pad "46" thru_hole oval (at 10.16 5.08 270) (size 1.7 1.7) (drill 1) (layers "*.Cu" "*.Mask") (remove_unused_layers no) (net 46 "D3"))
  (pad "47" thru_hole oval (at 7.62 5.08 270) (size 1.7 1.7) (drill 1) (layers "*.Cu" "*.Mask") (remove_unused_layers no) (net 47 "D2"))
  (pad "48" thru_hole oval (at 5.08 5.08 270) (size 1.7 1.7) (drill 1) (layers "*.Cu" "*.Mask") (remove_unused_layers no) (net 48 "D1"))
  (pad "49" thru_hole oval (at 2.54 5.08 270) (size 1.7 1.7) (drill 1) (layers "*.Cu" "*.Mask") (remove_unused_layers no) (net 49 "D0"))
  (pad "50" thru_hole oval (at 0 5.08 270) (size 1.7 1.7) (drill 1) (layers "*.Cu" "*.Mask") (remove_unused_layers no) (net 50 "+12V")))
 (gr_line (start 78.016 61.652) (end 195.491 61.652) (stroke (width 0.05) (type default)) (layer "Edge.Cuts"))
 (gr_line (start 195.539 121.473) (end 163.736 121.407) (stroke (width 0.05) (type default)) (layer "Edge.Cuts"))
 (gr_line (start 195.491 61.652) (end 195.539 121.473) (stroke (width 0.05) (type default)) (layer "Edge.Cuts"))
 (gr_line (start 98.004 121.428) (end 78.016 121.4305) (stroke (width 0.05) (type default)) (layer "Edge.Cuts"))
 (gr_line (start 78.016 121.4305) (end 78.016 61.652) (stroke (width 0.05) (type default)) (layer "Edge.Cuts"))
 (segment (start 108.658 107.609) (end 107.507 106.458) (width 0.2) (layer "B.Cu") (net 47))
 (segment (start 107.507 106.458) (end 107.507 91.275) (width 0.2) (layer "B.Cu") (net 47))
 (segment (start 107.507 91.275) (end 108.658 90.124) (width 0.2) (layer "B.Cu") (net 47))
 (segment (start 156.918 107.609) (end 155.767 106.458) (width 0.2) (layer "B.Cu") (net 28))
 (segment (start 155.767 106.458) (end 155.767 91.275) (width 0.2) (layer "B.Cu") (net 28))
 (segment (start 155.767 91.275) (end 156.918 90.124) (width 0.2) (layer "B.Cu") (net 28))
 (segment (start 125.287 106.458) (end 125.287 91.275) (width 0.2) (layer "B.Cu") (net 40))
 (segment (start 125.287 91.275) (end 126.438 90.124) (width 0.2) (layer "B.Cu") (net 40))
 (segment (start 126.438 107.609) (end 125.287 106.458) (width 0.2) (layer "B.Cu") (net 40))
 (segment (start 143.067 91.275) (end 144.218 90.124) (width 0.2) (layer "B.Cu") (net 33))
 (segment (start 144.218 107.609) (end 143.067 106.458) (width 0.2) (layer "B.Cu") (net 33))
 (segment (start 143.067 106.458) (end 143.067 91.275) (width 0.2) (layer "B.Cu") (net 33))
 (segment (start 148.147 106.458) (end 148.147 91.275) (width 0.2) (layer "B.Cu") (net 31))
 (segment (start 149.298 107.609) (end 148.147 106.458) (width 0.2) (layer "B.Cu") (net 31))
 (segment (start 148.147 91.275) (end 149.298 90.124) (width 0.2) (layer "B.Cu") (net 31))
 (segment (start 151.838 102.529) (end 151.838 95.204) (width 0.2) (layer "B.Cu") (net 21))
 (segment (start 141.678 102.529) (end 141.678 95.204) (width 0.2) (layer "B.Cu") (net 17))
 (segment (start 113.738 102.529) (end 113.738 95.204) (width 0.2) (layer "B.Cu") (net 6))
 (segment (start 103.578 107.609) (end 102.427 106.458) (width 0.2) (layer "B.Cu") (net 49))
 (segment (start 102.427 106.458) (end 102.427 91.275) (width 0.2) (layer "B.Cu") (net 49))
 (segment (start 102.427 91.275) (end 103.578 90.124) (width 0.2) (layer "B.Cu") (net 49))
 (segment (start 123.898 102.529) (end 123.898 95.204) (width 0.2) (layer "B.Cu") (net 10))
 (segment (start 150.687 106.458) (end 150.687 91.275) (width 0.2) (layer "B.Cu") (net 30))
 (segment (start 151.838 107.609) (end 150.687 106.458) (width 0.2) (layer "B.Cu") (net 30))
 (segment (start 150.687 91.275) (end 151.838 90.124) (width 0.2) (layer "B.Cu") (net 30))
 (segment (start 127.827 91.275) (end 128.978 90.124) (width 0.2) (layer "B.Cu") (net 39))
 (segment (start 127.827 106.458) (end 127.827 91.275) (width 0.2) (layer "B.Cu") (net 39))
 (segment (start 128.978 107.609) (end 127.827 106.458) (width 0.2) (layer "B.Cu") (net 39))
 (segment (start 115.127 91.275) (end 116.278 90.124) (width 0.2) (layer "B.Cu") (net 44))
 (segment (start 115.127 106.458) (end 115.127 91.275) (width 0.2) (layer "B.Cu") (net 44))
 (segment (start 116.278 107.609) (end 115.127 106.458) (width 0.2) (layer "B.Cu") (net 44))
 (segment (start 134.058 102.529) (end 134.058 95.204) (width 0.2) (layer "B.Cu") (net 14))
 (segment (start 153.227 91.275) (end 154.378 90.124) (width 0.2) (layer "B.Cu") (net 29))
 (segment (start 154.378 107.609) (end 153.227 106.458) (width 0.2) (layer "B.Cu") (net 29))
 (segment (start 153.227 106.458) (end 153.227 91.275) (width 0.2) (layer "B.Cu") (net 29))
 (segment (start 144.218 102.529) (end 144.218 95.204) (width 0.2) (layer "B.Cu") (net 18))
 (segment (start 106.118 102.529) (end 106.118 95.204) (width 0.2) (layer "B.Cu") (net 3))
 (segment (start 101.038 102.529) (end 101.038 95.204) (width 0.2) (layer "B.Cu") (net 1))
 (segment (start 117.667 106.458) (end 117.667 91.275) (width 0.2) (layer "B.Cu") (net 43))
 (segment (start 118.818 107.609) (end 117.667 106.458) (width 0.2) (layer "B.Cu") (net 43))
 (segment (start 117.667 91.275) (end 118.818 90.124) (width 0.2) (layer "B.Cu") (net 43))
 (segment (start 132.907 91.275) (end 134.058 90.124) (width 0.2) (layer "B.Cu") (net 37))
 (segment (start 132.907 106.458) (end 132.907 91.275) (width 0.2) (layer "B.Cu") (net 37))
 (segment (start 134.058 107.609) (end 132.907 106.458) (width 0.2) (layer "B.Cu") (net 37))
 (segment (start 131.518 107.609) (end 130.367 106.458) (width 0.2) (layer "B.Cu") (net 38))
 (segment (start 130.367 91.275) (end 131.518 90.124) (width 0.2) (layer "B.Cu") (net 38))
 (segment (start 130.367 106.458) (end 130.367 91.275) (width 0.2) (layer "B.Cu") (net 38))
 (segment (start 135.447 106.458) (end 135.447 91.275) (width 0.2) (layer "B.Cu") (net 36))
 (segment (start 136.598 107.609) (end 135.447 106.458) (width 0.2) (layer "B.Cu") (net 36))
 (segment (start 135.447 91.275) (end 136.598 90.124) (width 0.2) (layer "B.Cu") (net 36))
 (segment (start 126.438 102.529) (end 126.438 95.204) (width 0.2) (layer "B.Cu") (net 11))
 (segment (start 158.307 106.458) (end 158.307 91.275) (width 0.2) (layer "B.Cu") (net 27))
 (segment (start 158.307 91.275) (end 159.458 90.124) (width 0.2) (layer "B.Cu") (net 27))
 (segment (start 159.458 107.609) (end 158.307 106.458) (width 0.2) (layer "B.Cu") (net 27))
 (segment (start 120.207 91.275) (end 121.358 90.124) (width 0.2) (layer "B.Cu") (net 42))
 (segment (start 120.207 106.458) (end 120.207 91.275) (width 0.2) (layer "B.Cu") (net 42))
 (segment (start 121.358 107.609) (end 120.207 106.458) (width 0.2) (layer "B.Cu") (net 42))
 (segment (start 154.378 102.529) (end 154.378 95.204) (width 0.2) (layer "B.Cu") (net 22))
 (segment (start 103.578 102.529) (end 103.578 95.204) (width 0.2) (layer "B.Cu") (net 2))
 (segment (start 131.518 102.529) (end 131.518 95.204) (width 0.2) (layer "B.Cu") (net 13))
 (segment (start 128.978 102.529) (end 128.978 95.204) (width 0.2) (layer "B.Cu") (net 12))
 (segment (start 139.138 102.529) (end 139.138 95.204) (width 0.2) (layer "B.Cu") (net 16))
 (segment (start 104.967 106.458) (end 104.967 91.275) (width 0.2) (layer "B.Cu") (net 48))
 (segment (start 106.118 107.609) (end 104.967 106.458) (width 0.2) (layer "B.Cu") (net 48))
 (segment (start 104.967 91.275) (end 106.118 90.124) (width 0.2) (layer "B.Cu") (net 48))
 (segment (start 139.138 107.609) (end 137.987 106.458) (width 0.2) (layer "B.Cu") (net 35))
 (segment (start 137.987 106.458) (end 137.987 91.275) (width 0.2) (layer "B.Cu") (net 35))
 (segment (start 137.987 91.275) (end 139.138 90.124) (width 0.2) (layer "B.Cu") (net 35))
 (segment (start 146.758 102.529) (end 146.758 95.204) (width 0.2) (layer "B.Cu") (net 19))
 (segment (start 108.658 102.529) (end 108.658 95.204) (width 0.2) (layer "B.Cu") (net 4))
 (segment (start 161.998 107.609) (end 160.847 106.458) (width 0.2) (layer "B.Cu") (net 26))
 (segment (start 160.847 91.275) (end 161.998 90.124) (width 0.2) (layer "B.Cu") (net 26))
 (segment (start 160.847 106.458) (end 160.847 91.275) (width 0.2) (layer "B.Cu") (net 26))
 (segment (start 141.678 107.609) (end 140.527 106.458) (width 0.2) (layer "B.Cu") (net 34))
 (segment (start 140.527 91.275) (end 141.678 90.124) (width 0.2) (layer "B.Cu") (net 34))
 (segment (start 140.527 106.458) (end 140.527 91.275) (width 0.2) (layer "B.Cu") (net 34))
 (segment (start 122.747 106.458) (end 122.747 91.275) (width 0.2) (layer "B.Cu") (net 41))
 (segment (start 122.747 91.275) (end 123.898 90.124) (width 0.2) (layer "B.Cu") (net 41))
 (segment (start 123.898 107.609) (end 122.747 106.458) (width 0.2) (layer "B.Cu") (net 41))
 (segment (start 156.918 102.529) (end 156.918 95.204) (width 0.2) (layer "B.Cu") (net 23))
 (segment (start 101.038 107.609) (end 99.887 106.458) (width 0.2) (layer "B.Cu") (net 50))
 (segment (start 99.887 106.458) (end 99.887 91.275) (width 0.2) (layer "B.Cu") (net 50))
 (segment (start 99.887 91.275) (end 101.038 90.124) (width 0.2) (layer "B.Cu") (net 50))
 (segment (start 159.458 102.529) (end 159.458 95.204) (width 0.2) (layer "B.Cu") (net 24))
 (segment (start 145.607 91.275) (end 146.758 90.124) (width 0.2) (layer "B.Cu") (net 32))
 (segment (start 146.758 107.609) (end 145.607 106.458) (width 0.2) (layer "B.Cu") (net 32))
 (segment (start 145.607 106.458) (end 145.607 91.275) (width 0.2) (layer "B.Cu") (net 32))
 (segment (start 112.587 106.458) (end 112.587 91.275) (width 0.2) (layer "B.Cu") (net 45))
 (segment (start 112.587 91.275) (end 113.738 90.124) (width 0.2) (layer "B.Cu") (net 45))
 (segment (start 113.738 107.609) (end 112.587 106.458) (width 0.2) (layer "B.Cu") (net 45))
 (segment (start 161.998 102.529) (end 161.998 95.204) (width 0.2) (layer "B.Cu") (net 25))
 (segment (start 111.198 102.529) (end 111.198 95.204) (width 0.2) (layer "B.Cu") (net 5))
 (segment (start 136.598 102.529) (end 136.598 95.204) (width 0.2) (layer "B.Cu") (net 15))
 (segment (start 116.278 102.529) (end 116.278 95.204) (width 0.2) (layer "B.Cu") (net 7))
 (segment (start 121.358 102.529) (end 121.358 95.204) (width 0.2) (layer "B.Cu") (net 9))
 (segment (start 110.047 106.458) (end 110.047 91.275) (width 0.2) (layer "B.Cu") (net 46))
 (segment (start 110.047 91.275) (end 111.198 90.124) (width 0.2) (layer "B.Cu") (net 46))
 (segment (start 111.198 107.609) (end 110.047 106.458) (width 0.2) (layer "B.Cu") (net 46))
 (segment (start 149.298 102.529) (end 149.298 95.204) (width 0.2) (layer "B.Cu") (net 20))
 (segment (start 118.818 102.529) (end 118.818 95.204) (width 0.2) (layer "B.Cu") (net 8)))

